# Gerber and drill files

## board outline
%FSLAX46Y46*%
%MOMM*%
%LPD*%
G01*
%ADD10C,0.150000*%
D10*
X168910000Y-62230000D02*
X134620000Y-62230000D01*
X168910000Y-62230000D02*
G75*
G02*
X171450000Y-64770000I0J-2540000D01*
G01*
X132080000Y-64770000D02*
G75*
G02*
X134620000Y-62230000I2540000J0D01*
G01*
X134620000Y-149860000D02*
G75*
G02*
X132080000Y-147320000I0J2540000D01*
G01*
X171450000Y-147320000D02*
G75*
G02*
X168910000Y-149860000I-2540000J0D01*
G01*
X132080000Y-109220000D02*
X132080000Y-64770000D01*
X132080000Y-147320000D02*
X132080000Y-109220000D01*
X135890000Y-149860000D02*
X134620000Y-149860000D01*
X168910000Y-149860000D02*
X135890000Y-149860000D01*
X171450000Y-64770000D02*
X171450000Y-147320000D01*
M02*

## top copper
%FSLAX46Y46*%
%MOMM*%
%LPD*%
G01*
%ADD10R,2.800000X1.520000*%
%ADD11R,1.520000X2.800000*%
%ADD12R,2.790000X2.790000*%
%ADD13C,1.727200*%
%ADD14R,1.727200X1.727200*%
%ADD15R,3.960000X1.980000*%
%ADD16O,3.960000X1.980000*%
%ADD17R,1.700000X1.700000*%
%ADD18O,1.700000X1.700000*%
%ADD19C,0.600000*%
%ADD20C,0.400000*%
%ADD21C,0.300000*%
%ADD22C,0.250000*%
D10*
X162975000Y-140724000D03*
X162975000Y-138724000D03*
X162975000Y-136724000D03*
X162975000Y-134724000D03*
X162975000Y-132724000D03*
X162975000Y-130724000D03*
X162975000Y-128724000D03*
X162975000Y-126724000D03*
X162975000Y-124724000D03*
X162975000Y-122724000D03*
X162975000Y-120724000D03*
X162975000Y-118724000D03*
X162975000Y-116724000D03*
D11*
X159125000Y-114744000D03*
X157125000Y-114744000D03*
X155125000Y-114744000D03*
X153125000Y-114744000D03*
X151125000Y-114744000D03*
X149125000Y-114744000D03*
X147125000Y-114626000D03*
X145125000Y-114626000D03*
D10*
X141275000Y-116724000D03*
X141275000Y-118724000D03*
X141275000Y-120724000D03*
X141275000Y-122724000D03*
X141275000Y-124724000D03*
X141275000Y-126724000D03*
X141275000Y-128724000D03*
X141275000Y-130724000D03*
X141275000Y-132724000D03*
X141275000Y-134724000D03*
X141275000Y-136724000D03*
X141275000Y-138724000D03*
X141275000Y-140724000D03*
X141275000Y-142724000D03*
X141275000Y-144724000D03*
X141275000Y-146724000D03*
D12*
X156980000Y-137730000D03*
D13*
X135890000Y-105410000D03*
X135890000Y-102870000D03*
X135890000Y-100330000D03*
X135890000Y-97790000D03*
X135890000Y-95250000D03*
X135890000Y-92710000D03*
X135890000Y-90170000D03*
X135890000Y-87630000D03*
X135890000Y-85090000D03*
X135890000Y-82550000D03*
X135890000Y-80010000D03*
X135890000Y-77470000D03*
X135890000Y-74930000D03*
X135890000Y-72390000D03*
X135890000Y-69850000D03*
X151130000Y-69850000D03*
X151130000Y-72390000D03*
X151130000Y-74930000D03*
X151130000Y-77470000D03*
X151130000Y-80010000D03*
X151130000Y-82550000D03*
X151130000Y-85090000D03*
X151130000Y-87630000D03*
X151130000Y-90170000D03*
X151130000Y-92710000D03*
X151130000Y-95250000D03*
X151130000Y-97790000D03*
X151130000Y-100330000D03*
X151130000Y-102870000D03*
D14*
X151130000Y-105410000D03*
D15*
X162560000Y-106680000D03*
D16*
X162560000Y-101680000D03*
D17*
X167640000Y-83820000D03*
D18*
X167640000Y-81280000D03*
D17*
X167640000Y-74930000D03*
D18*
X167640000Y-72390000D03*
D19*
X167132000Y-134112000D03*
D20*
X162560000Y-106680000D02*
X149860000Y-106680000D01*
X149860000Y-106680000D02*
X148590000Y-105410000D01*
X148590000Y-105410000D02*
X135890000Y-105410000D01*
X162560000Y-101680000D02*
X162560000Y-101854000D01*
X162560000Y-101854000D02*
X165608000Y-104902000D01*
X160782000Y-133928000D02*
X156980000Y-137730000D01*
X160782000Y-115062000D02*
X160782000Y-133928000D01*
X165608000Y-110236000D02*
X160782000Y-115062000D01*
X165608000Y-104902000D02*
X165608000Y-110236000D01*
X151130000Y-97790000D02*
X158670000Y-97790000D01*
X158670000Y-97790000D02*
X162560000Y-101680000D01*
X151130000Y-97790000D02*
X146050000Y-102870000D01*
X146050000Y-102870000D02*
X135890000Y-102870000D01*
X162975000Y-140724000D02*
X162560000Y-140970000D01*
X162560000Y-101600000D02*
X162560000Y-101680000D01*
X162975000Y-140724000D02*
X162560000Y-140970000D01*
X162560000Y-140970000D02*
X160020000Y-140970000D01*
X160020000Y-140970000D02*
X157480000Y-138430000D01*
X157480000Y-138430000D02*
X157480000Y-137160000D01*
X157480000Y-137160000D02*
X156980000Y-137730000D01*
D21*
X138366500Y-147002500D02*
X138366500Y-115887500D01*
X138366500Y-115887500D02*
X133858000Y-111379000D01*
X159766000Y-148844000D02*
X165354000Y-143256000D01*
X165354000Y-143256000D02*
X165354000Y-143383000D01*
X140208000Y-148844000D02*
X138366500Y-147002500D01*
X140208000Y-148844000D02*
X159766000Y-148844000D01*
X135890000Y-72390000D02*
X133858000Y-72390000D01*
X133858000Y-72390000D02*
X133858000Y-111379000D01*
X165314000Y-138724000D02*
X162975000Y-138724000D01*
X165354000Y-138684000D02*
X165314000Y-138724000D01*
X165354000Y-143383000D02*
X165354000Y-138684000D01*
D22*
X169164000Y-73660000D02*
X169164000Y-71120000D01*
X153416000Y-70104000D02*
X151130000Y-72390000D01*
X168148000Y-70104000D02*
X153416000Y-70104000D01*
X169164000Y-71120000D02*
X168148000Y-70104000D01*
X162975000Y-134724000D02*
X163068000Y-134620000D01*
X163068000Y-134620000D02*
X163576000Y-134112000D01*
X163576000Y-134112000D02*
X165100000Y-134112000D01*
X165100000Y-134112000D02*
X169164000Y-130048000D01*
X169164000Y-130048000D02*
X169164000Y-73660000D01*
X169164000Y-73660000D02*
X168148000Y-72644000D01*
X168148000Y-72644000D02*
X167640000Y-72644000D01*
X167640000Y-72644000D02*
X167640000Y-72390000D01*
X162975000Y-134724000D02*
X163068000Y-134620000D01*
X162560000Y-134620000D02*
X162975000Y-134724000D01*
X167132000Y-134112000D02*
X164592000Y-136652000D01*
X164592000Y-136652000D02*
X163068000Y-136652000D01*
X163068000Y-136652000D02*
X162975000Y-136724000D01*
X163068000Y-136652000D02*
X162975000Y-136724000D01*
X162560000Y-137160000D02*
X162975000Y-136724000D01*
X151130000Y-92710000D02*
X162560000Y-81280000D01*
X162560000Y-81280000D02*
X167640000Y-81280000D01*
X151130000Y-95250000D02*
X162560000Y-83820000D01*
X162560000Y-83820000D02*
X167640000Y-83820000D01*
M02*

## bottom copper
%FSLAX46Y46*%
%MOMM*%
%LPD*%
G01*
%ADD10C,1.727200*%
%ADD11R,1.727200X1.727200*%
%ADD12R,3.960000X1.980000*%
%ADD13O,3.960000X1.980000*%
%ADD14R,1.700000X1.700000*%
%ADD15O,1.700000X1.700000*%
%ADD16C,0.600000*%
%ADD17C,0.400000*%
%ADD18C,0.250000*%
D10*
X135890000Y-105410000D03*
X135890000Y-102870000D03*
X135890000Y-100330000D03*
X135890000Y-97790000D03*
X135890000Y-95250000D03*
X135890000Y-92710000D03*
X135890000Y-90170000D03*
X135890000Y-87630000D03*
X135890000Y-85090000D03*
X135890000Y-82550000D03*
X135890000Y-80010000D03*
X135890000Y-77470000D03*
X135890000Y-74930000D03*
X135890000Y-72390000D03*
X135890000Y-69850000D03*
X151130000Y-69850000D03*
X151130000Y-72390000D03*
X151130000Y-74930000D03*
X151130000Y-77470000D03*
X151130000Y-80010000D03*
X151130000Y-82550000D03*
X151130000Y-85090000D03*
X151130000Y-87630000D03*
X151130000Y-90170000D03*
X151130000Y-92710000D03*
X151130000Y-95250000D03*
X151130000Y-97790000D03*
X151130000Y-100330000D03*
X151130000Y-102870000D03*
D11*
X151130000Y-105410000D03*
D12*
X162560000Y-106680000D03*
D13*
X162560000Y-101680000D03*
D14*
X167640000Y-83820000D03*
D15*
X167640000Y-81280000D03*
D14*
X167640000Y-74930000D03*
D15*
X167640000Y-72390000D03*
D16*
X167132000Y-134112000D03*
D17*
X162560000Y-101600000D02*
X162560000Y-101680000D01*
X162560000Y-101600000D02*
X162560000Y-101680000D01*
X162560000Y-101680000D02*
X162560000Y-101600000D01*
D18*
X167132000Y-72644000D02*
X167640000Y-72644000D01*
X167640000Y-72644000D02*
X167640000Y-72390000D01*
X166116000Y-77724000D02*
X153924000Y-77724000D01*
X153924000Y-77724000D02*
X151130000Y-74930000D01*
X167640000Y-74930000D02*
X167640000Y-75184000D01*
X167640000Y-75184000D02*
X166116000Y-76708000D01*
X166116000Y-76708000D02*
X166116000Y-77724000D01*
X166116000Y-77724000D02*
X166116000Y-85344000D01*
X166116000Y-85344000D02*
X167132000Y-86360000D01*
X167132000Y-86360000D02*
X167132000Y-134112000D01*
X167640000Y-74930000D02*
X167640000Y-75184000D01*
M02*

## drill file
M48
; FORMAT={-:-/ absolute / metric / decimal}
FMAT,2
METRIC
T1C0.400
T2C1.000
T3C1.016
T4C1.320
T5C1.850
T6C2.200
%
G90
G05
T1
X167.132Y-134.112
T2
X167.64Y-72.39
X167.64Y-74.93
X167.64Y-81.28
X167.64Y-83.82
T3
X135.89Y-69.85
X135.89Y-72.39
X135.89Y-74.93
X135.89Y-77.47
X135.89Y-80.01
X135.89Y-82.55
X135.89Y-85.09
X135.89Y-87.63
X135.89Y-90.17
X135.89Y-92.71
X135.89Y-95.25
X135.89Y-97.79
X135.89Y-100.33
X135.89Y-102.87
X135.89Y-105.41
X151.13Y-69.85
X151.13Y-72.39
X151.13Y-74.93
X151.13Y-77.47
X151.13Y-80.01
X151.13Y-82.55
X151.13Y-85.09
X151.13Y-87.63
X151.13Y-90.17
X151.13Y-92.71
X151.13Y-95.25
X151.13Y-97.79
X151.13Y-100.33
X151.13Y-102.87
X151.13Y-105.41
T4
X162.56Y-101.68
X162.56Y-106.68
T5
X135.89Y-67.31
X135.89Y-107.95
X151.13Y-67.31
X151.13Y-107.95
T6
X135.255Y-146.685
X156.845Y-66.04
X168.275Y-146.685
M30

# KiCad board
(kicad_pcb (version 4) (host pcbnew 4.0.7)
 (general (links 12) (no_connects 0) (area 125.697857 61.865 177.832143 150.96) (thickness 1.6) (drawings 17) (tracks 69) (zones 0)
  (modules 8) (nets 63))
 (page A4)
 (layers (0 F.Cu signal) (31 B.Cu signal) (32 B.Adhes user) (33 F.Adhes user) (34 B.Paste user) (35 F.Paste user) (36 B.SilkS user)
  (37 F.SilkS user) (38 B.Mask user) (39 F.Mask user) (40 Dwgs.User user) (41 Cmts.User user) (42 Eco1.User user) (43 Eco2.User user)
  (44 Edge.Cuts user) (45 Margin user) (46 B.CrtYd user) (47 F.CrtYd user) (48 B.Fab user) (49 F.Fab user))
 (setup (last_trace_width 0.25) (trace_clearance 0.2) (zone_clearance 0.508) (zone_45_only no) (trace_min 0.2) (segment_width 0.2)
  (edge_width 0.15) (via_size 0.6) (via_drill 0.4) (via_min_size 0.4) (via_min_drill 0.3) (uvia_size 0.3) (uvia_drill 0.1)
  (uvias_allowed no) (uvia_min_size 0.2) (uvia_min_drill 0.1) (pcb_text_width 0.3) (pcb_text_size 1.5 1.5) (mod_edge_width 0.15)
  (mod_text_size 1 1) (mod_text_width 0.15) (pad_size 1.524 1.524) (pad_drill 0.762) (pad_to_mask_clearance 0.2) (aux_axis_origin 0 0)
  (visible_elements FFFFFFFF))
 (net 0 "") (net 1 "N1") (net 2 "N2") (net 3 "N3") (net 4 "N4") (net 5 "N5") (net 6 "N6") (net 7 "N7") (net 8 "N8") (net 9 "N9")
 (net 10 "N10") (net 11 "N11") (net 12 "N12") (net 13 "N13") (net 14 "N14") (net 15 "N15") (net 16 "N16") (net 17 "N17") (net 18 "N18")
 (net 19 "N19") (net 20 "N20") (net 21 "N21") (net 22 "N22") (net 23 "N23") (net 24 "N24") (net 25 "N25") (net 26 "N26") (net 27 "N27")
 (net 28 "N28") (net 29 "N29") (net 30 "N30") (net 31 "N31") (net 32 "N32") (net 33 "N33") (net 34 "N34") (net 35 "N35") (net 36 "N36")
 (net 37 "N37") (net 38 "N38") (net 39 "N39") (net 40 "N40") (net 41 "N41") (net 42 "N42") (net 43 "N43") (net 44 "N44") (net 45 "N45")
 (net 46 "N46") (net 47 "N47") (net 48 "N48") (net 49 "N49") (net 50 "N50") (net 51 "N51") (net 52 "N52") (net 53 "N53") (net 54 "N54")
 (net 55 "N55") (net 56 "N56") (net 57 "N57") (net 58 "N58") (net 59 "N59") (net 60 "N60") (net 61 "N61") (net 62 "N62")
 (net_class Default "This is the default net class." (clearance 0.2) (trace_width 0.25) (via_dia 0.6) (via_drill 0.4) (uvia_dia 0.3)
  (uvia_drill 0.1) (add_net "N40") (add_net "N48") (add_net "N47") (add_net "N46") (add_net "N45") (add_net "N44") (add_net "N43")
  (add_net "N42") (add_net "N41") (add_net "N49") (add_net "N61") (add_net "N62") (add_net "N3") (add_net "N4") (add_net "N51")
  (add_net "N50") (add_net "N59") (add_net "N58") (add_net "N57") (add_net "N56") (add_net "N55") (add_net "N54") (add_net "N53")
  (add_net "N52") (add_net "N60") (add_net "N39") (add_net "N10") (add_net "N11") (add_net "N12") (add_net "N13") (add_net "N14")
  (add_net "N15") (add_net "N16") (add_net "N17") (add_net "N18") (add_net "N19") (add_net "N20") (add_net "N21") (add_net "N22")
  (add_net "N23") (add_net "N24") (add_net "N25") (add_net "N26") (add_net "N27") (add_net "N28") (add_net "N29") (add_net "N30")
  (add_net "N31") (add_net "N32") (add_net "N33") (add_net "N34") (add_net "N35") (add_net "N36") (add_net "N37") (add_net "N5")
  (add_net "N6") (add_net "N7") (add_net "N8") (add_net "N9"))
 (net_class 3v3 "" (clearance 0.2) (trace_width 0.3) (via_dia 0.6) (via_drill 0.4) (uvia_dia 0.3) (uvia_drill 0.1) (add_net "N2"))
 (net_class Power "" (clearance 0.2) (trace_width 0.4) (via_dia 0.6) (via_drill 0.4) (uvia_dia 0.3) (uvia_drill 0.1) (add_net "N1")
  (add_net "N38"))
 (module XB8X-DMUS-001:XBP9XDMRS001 (layer F.Cu) (at 152.4 130.81 180)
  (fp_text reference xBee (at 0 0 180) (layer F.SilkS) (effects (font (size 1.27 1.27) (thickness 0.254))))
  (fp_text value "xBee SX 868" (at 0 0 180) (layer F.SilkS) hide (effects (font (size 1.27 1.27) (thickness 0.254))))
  (pad 1 smd rect (at -10.575 -9.914 270) (size 1.52 2.8) (layers F.Cu F.Paste F.Mask) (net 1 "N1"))
  (pad 2 smd rect (at -10.575 -7.914 270) (size 1.52 2.8) (layers F.Cu F.Paste F.Mask) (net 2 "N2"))
  (pad 3 smd rect (at -10.575 -5.914 270) (size 1.52 2.8) (layers F.Cu F.Paste F.Mask) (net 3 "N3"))
  (pad 4 smd rect (at -10.575 -3.914 270) (size 1.52 2.8) (layers F.Cu F.Paste F.Mask) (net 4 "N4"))
  (pad 5 smd rect (at -10.575 -1.914 270) (size 1.52 2.8) (layers F.Cu F.Paste F.Mask) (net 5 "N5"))
  (pad 6 smd rect (at -10.575 0.086 270) (size 1.52 2.8) (layers F.Cu F.Paste F.Mask) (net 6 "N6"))
  (pad 7 smd rect (at -10.575 2.086 270) (size 1.52 2.8) (layers F.Cu F.Paste F.Mask) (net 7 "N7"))
  (pad 8 smd rect (at -10.575 4.086 270) (size 1.52 2.8) (layers F.Cu F.Paste F.Mask) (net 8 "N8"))
  (pad 9 smd rect (at -10.575 6.086 270) (size 1.52 2.8) (layers F.Cu F.Paste F.Mask) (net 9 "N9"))
  (pad 10 smd rect (at -10.575 8.086 270) (size 1.52 2.8) (layers F.Cu F.Paste F.Mask) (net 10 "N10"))
  (pad 11 smd rect (at -10.575 10.086 270) (size 1.52 2.8) (layers F.Cu F.Paste F.Mask) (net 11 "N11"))
  (pad 12 smd rect (at -10.575 12.086 270) (size 1.52 2.8) (layers F.Cu F.Paste F.Mask) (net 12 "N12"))
  (pad 13 smd rect (at -10.575 14.086 270) (size 1.52 2.8) (layers F.Cu F.Paste F.Mask) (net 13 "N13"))
  (pad 14 smd rect (at -6.725 16.066 180) (size 1.52 2.8) (layers F.Cu F.Paste F.Mask) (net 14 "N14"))
  (pad 15 smd rect (at -4.725 16.066 180) (size 1.52 2.8) (layers F.Cu F.Paste F.Mask) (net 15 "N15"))
  (pad 16 smd rect (at -2.725 16.066 180) (size 1.52 2.8) (layers F.Cu F.Paste F.Mask) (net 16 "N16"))
  (pad 17 smd rect (at -0.725 16.066 180) (size 1.52 2.8) (layers F.Cu F.Paste F.Mask) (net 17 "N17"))
  (pad 18 smd rect (at 1.275 16.066 180) (size 1.52 2.8) (layers F.Cu F.Paste F.Mask) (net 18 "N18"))
  (pad 19 smd rect (at 3.275 16.066 180) (size 1.52 2.8) (layers F.Cu F.Paste F.Mask) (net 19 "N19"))
  (pad 20 smd rect (at 5.275 16.184 180) (size 1.52 2.8) (layers F.Cu F.Paste F.Mask) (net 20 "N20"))
  (pad 21 smd rect (at 7.275 16.184 180) (size 1.52 2.8) (layers F.Cu F.Paste F.Mask) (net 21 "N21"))
  (pad 22 smd rect (at 11.125 14.086 270) (size 1.52 2.8) (layers F.Cu F.Paste F.Mask) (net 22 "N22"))
  (pad 23 smd rect (at 11.125 12.086 270) (size 1.52 2.8) (layers F.Cu F.Paste F.Mask) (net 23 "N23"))
  (pad 24 smd rect (at 11.125 10.086 270) (size 1.52 2.8) (layers F.Cu F.Paste F.Mask) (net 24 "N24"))
  (pad 25 smd rect (at 11.125 8.086 270) (size 1.52 2.8) (layers F.Cu F.Paste F.Mask) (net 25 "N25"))
  (pad 26 smd rect (at 11.125 6.086 270) (size 1.52 2.8) (layers F.Cu F.Paste F.Mask) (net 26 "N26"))
  (pad 27 smd rect (at 11.125 4.086 270) (size 1.52 2.8) (layers F.Cu F.Paste F.Mask) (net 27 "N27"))
  (pad 28 smd rect (at 11.125 2.086 270) (size 1.52 2.8) (layers F.Cu F.Paste F.Mask) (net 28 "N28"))
  (pad 29 smd rect (at 11.125 0.086 270) (size 1.52 2.8) (layers F.Cu F.Paste F.Mask) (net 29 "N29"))
  (pad 30 smd rect (at 11.125 -1.914 270) (size 1.52 2.8) (layers F.Cu F.Paste F.Mask) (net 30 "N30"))
  (pad 31 smd rect (at 11.125 -3.914 270) (size 1.52 2.8) (layers F.Cu F.Paste F.Mask) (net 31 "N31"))
  (pad 32 smd rect (at 11.125 -5.914 270) (size 1.52 2.8) (layers F.Cu F.Paste F.Mask) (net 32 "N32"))
  (pad 33 smd rect (at 11.125 -7.914 270) (size 1.52 2.8) (layers F.Cu F.Paste F.Mask) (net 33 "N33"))
  (pad 34 smd rect (at 11.125 -9.914 270) (size 1.52 2.8) (layers F.Cu F.Paste F.Mask) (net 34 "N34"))
  (pad 35 smd rect (at 11.125 -11.914 270) (size 1.52 2.8) (layers F.Cu F.Paste F.Mask) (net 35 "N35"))
  (pad 36 smd rect (at 11.125 -13.914 270) (size 1.52 2.8) (layers F.Cu F.Paste F.Mask) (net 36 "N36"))
  (pad 37 smd rect (at 11.125 -15.914 270) (size 1.52 2.8) (layers F.Cu F.Paste F.Mask) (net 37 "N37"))
  (pad 38 smd rect (at -4.58 -6.92 180) (size 2.79 2.79) (layers F.Cu F.Paste F.Mask) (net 1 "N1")))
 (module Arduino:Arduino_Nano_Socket (layer F.Cu) (at 143.51 66.04 180)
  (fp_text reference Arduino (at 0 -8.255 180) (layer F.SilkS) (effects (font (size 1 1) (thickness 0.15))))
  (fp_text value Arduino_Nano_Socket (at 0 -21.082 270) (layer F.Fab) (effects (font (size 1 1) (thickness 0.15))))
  (pad VIN thru_hole circle (at 7.62 -39.37 180) (size 1.7272 1.7272) (drill 1.016) (layers *.Cu *.Mask) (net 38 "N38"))
  (pad GND2 thru_hole circle (at 7.62 -36.83 180) (size 1.7272 1.7272) (drill 1.016) (layers *.Cu *.Mask) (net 1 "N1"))
  (pad RST2 thru_hole circle (at 7.62 -34.29 180) (size 1.7272 1.7272) (drill 1.016) (layers *.Cu *.Mask) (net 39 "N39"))
  (pad 5V thru_hole circle (at 7.62 -31.75 180) (size 1.7272 1.7272) (drill 1.016) (layers *.Cu *.Mask) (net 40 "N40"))
  (pad A7 thru_hole circle (at 7.62 -29.21 180) (size 1.7272 1.7272) (drill 1.016) (layers *.Cu *.Mask) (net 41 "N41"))
  (pad A6 thru_hole circle (at 7.62 -26.67 180) (size 1.7272 1.7272) (drill 1.016) (layers *.Cu *.Mask) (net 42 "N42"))
  (pad A5 thru_hole circle (at 7.62 -24.13 180) (size 1.7272 1.7272) (drill 1.016) (layers *.Cu *.Mask) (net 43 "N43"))
  (pad A4 thru_hole circle (at 7.62 -21.59 180) (size 1.7272 1.7272) (drill 1.016) (layers *.Cu *.Mask) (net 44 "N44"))
  (pad A3 thru_hole circle (at 7.62 -19.05 180) (size 1.7272 1.7272) (drill 1.016) (layers *.Cu *.Mask) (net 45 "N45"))
  (pad A2 thru_hole circle (at 7.62 -16.51 180) (size 1.7272 1.7272) (drill 1.016) (layers *.Cu *.Mask) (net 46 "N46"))
  (pad A1 thru_hole circle (at 7.62 -13.97 180) (size 1.7272 1.7272) (drill 1.016) (layers *.Cu *.Mask) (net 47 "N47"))
  (pad A0 thru_hole circle (at 7.62 -11.43 180) (size 1.7272 1.7272) (drill 1.016) (layers *.Cu *.Mask) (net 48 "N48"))
  (pad AREF thru_hole circle (at 7.62 -8.89 180) (size 1.7272 1.7272) (drill 1.016) (layers *.Cu *.Mask) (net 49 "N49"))
  (pad 3V3 thru_hole circle (at 7.62 -6.35 180) (size 1.7272 1.7272) (drill 1.016) (layers *.Cu *.Mask) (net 2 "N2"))
  (pad D13 thru_hole circle (at 7.62 -3.81 180) (size 1.7272 1.7272) (drill 1.016) (layers *.Cu *.Mask) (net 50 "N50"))
  (pad D12 thru_hole circle (at -7.62 -3.81 180) (size 1.7272 1.7272) (drill 1.016) (layers *.Cu *.Mask) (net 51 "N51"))
  (pad D11 thru_hole circle (at -7.62 -6.35 180) (size 1.7272 1.7272) (drill 1.016) (layers *.Cu *.Mask) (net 4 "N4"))
  (pad D10 thru_hole circle (at -7.62 -8.89 180) (size 1.7272 1.7272) (drill 1.016) (layers *.Cu *.Mask) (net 3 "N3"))
  (pad D9 thru_hole circle (at -7.62 -11.43 180) (size 1.7272 1.7272) (drill 1.016) (layers *.Cu *.Mask) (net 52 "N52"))
  (pad D8 thru_hole circle (at -7.62 -13.97 180) (size 1.7272 1.7272) (drill 1.016) (layers *.Cu *.Mask) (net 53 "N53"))
  (pad D7 thru_hole circle (at -7.62 -16.51 180) (size 1.7272 1.7272) (drill 1.016) (layers *.Cu *.Mask) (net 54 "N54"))
  (pad D6 thru_hole circle (at -7.62 -19.05 180) (size 1.7272 1.7272) (drill 1.016) (layers *.Cu *.Mask) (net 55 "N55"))
  (pad D5 thru_hole circle (at -7.62 -21.59 180) (size 1.7272 1.7272) (drill 1.016) (layers *.Cu *.Mask) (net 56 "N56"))
  (pad D4 thru_hole circle (at -7.62 -24.13 180) (size 1.7272 1.7272) (drill 1.016) (layers *.Cu *.Mask) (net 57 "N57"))
  (pad D3 thru_hole circle (at -7.62 -26.67 180) (size 1.7272 1.7272) (drill 1.016) (layers *.Cu *.Mask) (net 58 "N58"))
  (pad D2 thru_hole circle (at -7.62 -29.21 180) (size 1.7272 1.7272) (drill 1.016) (layers *.Cu *.Mask) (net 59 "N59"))
  (pad GND1 thru_hole circle (at -7.62 -31.75 180) (size 1.7272 1.7272) (drill 1.016) (layers *.Cu *.Mask) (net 1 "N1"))
  (pad RST1 thru_hole circle (at -7.62 -34.29 180) (size 1.7272 1.7272) (drill 1.016) (layers *.Cu *.Mask) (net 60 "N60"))
  (pad D0 thru_hole circle (at -7.62 -36.83 180) (size 1.7272 1.7272) (drill 1.016) (layers *.Cu *.Mask) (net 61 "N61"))
  (pad D1 thru_hole rect (at -7.62 -39.37 180) (size 1.7272 1.7272) (drill 1.016) (layers *.Cu *.Mask) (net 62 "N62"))
  (pad "" np_thru_hole circle (at -7.62 -41.91 180) (size 1.85 1.85) (drill 1.85) (layers *.Cu *.Mask))
  (pad "" np_thru_hole circle (at 7.62 -41.91 180) (size 1.85 1.85) (drill 1.85) (layers *.Cu *.Mask))
  (pad "" np_thru_hole circle (at -7.62 -1.27 180) (size 1.85 1.85) (drill 1.85) (layers *.Cu *.Mask))
  (pad "" np_thru_hole circle (at 7.62 -1.27 180) (size 1.85 1.85) (drill 1.85) (layers *.Cu *.Mask)))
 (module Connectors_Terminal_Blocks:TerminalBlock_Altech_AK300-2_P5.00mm (layer F.Cu) (at 162.56 106.68 90)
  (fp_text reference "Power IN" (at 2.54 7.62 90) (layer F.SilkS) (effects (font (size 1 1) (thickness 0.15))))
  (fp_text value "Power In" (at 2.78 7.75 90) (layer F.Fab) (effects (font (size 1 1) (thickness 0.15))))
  (pad 1 thru_hole rect (at 0 0 90) (size 1.98 3.96) (drill 1.32) (layers *.Cu *.Mask) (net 38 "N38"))
  (pad 2 thru_hole oval (at 5 0 90) (size 1.98 3.96) (drill 1.32) (layers *.Cu *.Mask) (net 1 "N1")))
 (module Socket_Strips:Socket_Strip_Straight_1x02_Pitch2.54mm (layer F.Cu) (at 167.64 83.82 180)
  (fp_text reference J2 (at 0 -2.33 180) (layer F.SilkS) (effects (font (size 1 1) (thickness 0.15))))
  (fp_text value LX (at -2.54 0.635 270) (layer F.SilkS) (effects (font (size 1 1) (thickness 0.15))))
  (pad 1 thru_hole rect (at 0 0 180) (size 1.7 1.7) (drill 1) (layers *.Cu *.Mask) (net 59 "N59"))
  (pad 2 thru_hole oval (at 0 2.54 180) (size 1.7 1.7) (drill 1) (layers *.Cu *.Mask) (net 58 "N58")))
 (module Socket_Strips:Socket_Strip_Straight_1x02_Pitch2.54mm (layer F.Cu) (at 167.64 74.93 180)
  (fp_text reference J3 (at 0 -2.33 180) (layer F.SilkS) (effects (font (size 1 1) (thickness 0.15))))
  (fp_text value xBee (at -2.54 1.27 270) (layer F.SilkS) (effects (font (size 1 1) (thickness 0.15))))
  (pad 1 thru_hole rect (at 0 0 180) (size 1.7 1.7) (drill 1) (layers *.Cu *.Mask) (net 3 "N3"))
  (pad 2 thru_hole oval (at 0 2.54 180) (size 1.7 1.7) (drill 1) (layers *.Cu *.Mask) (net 4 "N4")))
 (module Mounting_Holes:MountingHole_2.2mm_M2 (layer F.Cu) (at 168.275 146.685)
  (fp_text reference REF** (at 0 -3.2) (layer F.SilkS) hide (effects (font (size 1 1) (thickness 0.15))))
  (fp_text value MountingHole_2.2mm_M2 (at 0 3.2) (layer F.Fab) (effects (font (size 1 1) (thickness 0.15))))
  (pad 1 np_thru_hole circle (at 0 0) (size 2.2 2.2) (drill 2.2) (layers *.Cu *.Mask)))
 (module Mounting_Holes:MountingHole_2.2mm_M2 (layer F.Cu) (at 135.255 146.685)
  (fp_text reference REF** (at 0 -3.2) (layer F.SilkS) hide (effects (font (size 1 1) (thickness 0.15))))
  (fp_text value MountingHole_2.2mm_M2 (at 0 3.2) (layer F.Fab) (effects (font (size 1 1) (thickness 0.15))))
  (pad 1 np_thru_hole circle (at 0 0) (size 2.2 2.2) (drill 2.2) (layers *.Cu *.Mask)))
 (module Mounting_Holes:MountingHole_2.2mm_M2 (layer F.Cu) (at 156.845 66.04)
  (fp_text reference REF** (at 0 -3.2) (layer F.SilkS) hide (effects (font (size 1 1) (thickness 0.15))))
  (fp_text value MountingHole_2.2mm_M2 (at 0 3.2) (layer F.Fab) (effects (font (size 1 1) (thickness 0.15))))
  (pad 1 np_thru_hole circle (at 0 0) (size 2.2 2.2) (drill 2.2) (layers *.Cu *.Mask)))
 (gr_line (start 168.91 62.23) (end 134.62 62.23) (angle 90) (layer Edge.Cuts) (width 0.15))
 (gr_arc (start 168.91 64.77) (end 168.91 62.23) (angle 90) (layer Edge.Cuts) (width 0.15))
 (gr_arc (start 134.62 64.77) (end 132.08 64.77) (angle 90) (layer Edge.Cuts) (width 0.15))
 (gr_arc (start 134.62 147.32) (end 134.62 149.86) (angle 90) (layer Edge.Cuts) (width 0.15))
 (gr_arc (start 168.91 147.32) (end 171.45 147.32) (angle 90) (layer Edge.Cuts) (width 0.15))
 (gr_line (start 132.08 109.22) (end 132.08 64.77) (angle 90) (layer Edge.Cuts) (width 0.15))
 (gr_line (start 132.08 147.32) (end 132.08 109.22) (angle 90) (layer Edge.Cuts) (width 0.15))
 (gr_line (start 135.89 149.86) (end 134.62 149.86) (angle 90) (layer Edge.Cuts) (width 0.15))
 (gr_line (start 168.91 149.86) (end 135.89 149.86) (angle 90) (layer Edge.Cuts) (width 0.15))
 (gr_line (start 171.45 64.77) (end 171.45 147.32) (angle 90) (layer Edge.Cuts) (width 0.15))
 (segment (start 162.56 106.68) (end 149.86 106.68) (width 0.4) (layer F.Cu) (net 38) (status 80000))
 (segment (start 149.86 106.68) (end 148.59 105.41) (width 0.4) (layer F.Cu) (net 38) (status 80000))
 (segment (start 148.59 105.41) (end 135.89 105.41) (width 0.4) (layer F.Cu) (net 38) (status 80000))
 (segment (start 162.56 101.68) (end 162.56 101.854) (width 0.4) (layer F.Cu) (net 1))
 (segment (start 162.56 101.854) (end 165.608 104.902) (width 0.4) (layer F.Cu) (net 1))
 (segment (start 160.782 133.928) (end 156.98 137.73) (width 0.4) (layer F.Cu) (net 1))
 (segment (start 160.782 115.062) (end 160.782 133.928) (width 0.4) (layer F.Cu) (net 1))
 (segment (start 165.608 110.236) (end 160.782 115.062) (width 0.4) (layer F.Cu) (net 1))
 (segment (start 165.608 104.902) (end 165.608 110.236) (width 0.4) (layer F.Cu) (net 1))
 (segment (start 151.13 97.79) (end 158.67 97.79) (width 0.4) (layer F.Cu) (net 1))
 (segment (start 158.67 97.79) (end 162.56 101.68) (width 0.4) (layer F.Cu) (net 1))
 (segment (start 162.56 101.6) (end 162.56 101.68) (width 0.4) (layer B.Cu) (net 1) (status 80000))
 (segment (start 151.13 97.79) (end 146.05 102.87) (width 0.4) (layer F.Cu) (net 1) (status 80000))
 (segment (start 146.05 102.87) (end 135.89 102.87) (width 0.4) (layer F.Cu) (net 1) (status 80000))
 (segment (start 162.56 101.6) (end 162.56 101.68) (width 0.4) (layer B.Cu) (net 1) (status 80000))
 (segment (start 162.975 140.724) (end 162.56 140.97) (width 0.4) (layer F.Cu) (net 1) (status 80000))
 (segment (start 162.56 101.6) (end 162.56 101.68) (width 0.4) (layer F.Cu) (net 1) (status 80000))
 (segment (start 162.56 101.68) (end 162.56 101.6) (width 0.4) (layer B.Cu) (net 1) (status 80000))
 (segment (start 162.975 140.724) (end 162.56 140.97) (width 0.4) (layer F.Cu) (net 1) (status 80000))
 (segment (start 162.56 140.97) (end 160.02 140.97) (width 0.4) (layer F.Cu) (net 1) (status 80000))
 (segment (start 160.02 140.97) (end 157.48 138.43) (width 0.4) (layer F.Cu) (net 1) (status 80000))
 (segment (start 157.48 138.43) (end 157.48 137.16) (width 0.4) (layer F.Cu) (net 1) (status 80000))
 (segment (start 157.48 137.16) (end 156.98 137.73) (width 0.4) (layer F.Cu) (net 1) (status 80000))
 (segment (start 138.3665 147.0025) (end 138.3665 115.8875) (width 0.3) (layer F.Cu) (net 2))
 (segment (start 138.3665 115.8875) (end 133.858 111.379) (width 0.3) (layer F.Cu) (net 2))
 (segment (start 159.766 148.844) (end 165.354 143.256) (width 0.3) (layer F.Cu) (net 2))
 (segment (start 165.354 143.256) (end 165.354 143.383) (width 0.3) (layer F.Cu) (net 2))
 (segment (start 140.208 148.844) (end 138.3665 147.0025) (width 0.3) (layer F.Cu) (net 2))
 (segment (start 140.208 148.844) (end 159.766 148.844) (width 0.3) (layer F.Cu) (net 2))
 (segment (start 135.89 72.39) (end 133.858 72.39) (width 0.3) (layer F.Cu) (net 2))
 (segment (start 133.858 72.39) (end 133.858 111.379) (width 0.3) (layer F.Cu) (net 2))
 (segment (start 165.314 138.724) (end 162.975 138.724) (width 0.3) (layer F.Cu) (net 2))
 (segment (start 165.354 138.684) (end 165.314 138.724) (width 0.3) (layer F.Cu) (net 2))
 (segment (start 165.354 143.383) (end 165.354 138.684) (width 0.3) (layer F.Cu) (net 2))
 (segment (start 169.164 73.66) (end 169.164 71.12) (width 0.25) (layer F.Cu) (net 4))
 (segment (start 153.416 70.104) (end 151.13 72.39) (width 0.25) (layer F.Cu) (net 4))
 (segment (start 168.148 70.104) (end 153.416 70.104) (width 0.25) (layer F.Cu) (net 4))
 (segment (start 169.164 71.12) (end 168.148 70.104) (width 0.25) (layer F.Cu) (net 4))
 (segment (start 162.975 134.724) (end 163.068 134.62) (width 0.25) (layer F.Cu) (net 4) (status 80000))
 (segment (start 163.068 134.62) (end 163.576 134.112) (width 0.25) (layer F.Cu) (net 4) (status 80000))
 (segment (start 163.576 134.112) (end 165.1 134.112) (width 0.25) (layer F.Cu) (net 4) (status 80000))
 (segment (start 165.1 134.112) (end 169.164 130.048) (width 0.25) (layer F.Cu) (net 4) (status 80000))
 (segment (start 169.164 130.048) (end 169.164 73.66) (width 0.25) (layer F.Cu) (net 4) (status 80000))
 (segment (start 169.164 73.66) (end 168.148 72.644) (width 0.25) (layer F.Cu) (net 4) (status 80000))
 (segment (start 168.148 72.644) (end 167.64 72.644) (width 0.25) (layer F.Cu) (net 4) (status 80000))
 (segment (start 167.64 72.644) (end 167.64 72.39) (width 0.25) (layer F.Cu) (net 4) (status 80000))
 (segment (start 162.975 134.724) (end 163.068 134.62) (width 0.25) (layer F.Cu) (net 4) (status 80000))
 (segment (start 167.132 72.644) (end 167.64 72.644) (width 0.25) (layer B.Cu) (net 4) (status 80000))
 (segment (start 167.64 72.644) (end 167.64 72.39) (width 0.25) (layer B.Cu) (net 4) (status 80000))
 (segment (start 162.56 134.62) (end 162.975 134.724) (width 0.25) (layer F.Cu) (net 4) (status 80000))
 (segment (start 166.116 77.724) (end 153.924 77.724) (width 0.25) (layer B.Cu) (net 3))
 (segment (start 153.924 77.724) (end 151.13 74.93) (width 0.25) (layer B.Cu) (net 3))
 (segment (start 167.64 74.93) (end 167.64 75.184) (width 0.25) (layer B.Cu) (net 3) (status 80000))
 (segment (start 167.64 75.184) (end 166.116 76.708) (width 0.25) (layer B.Cu) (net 3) (status 80000))
 (segment (start 166.116 76.708) (end 166.116 77.724) (width 0.25) (layer B.Cu) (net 3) (status 80000))
 (segment (start 166.116 77.724) (end 166.116 85.344) (width 0.25) (layer B.Cu) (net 3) (status 80000))
 (segment (start 166.116 85.344) (end 167.132 86.36) (width 0.25) (layer B.Cu) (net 3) (status 80000))
 (segment (start 167.132 86.36) (end 167.132 134.112) (width 0.25) (layer B.Cu) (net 3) (status 80000))
 (via (at 167.132 134.112) (size 0.6) (layers F.Cu B.Cu) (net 3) (status 80000))
 (segment (start 167.132 134.112) (end 164.592 136.652) (width 0.25) (layer F.Cu) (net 3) (status 80000))
 (segment (start 164.592 136.652) (end 163.068 136.652) (width 0.25) (layer F.Cu) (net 3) (status 80000))
 (segment (start 163.068 136.652) (end 162.975 136.724) (width 0.25) (layer F.Cu) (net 3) (status 80000))
 (segment (start 167.64 74.93) (end 167.64 75.184) (width 0.25) (layer B.Cu) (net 3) (status 80000))
 (segment (start 163.068 136.652) (end 162.975 136.724) (width 0.25) (layer F.Cu) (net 3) (status 80000))
 (segment (start 162.56 137.16) (end 162.975 136.724) (width 0.25) (layer F.Cu) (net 3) (status 80000))
 (segment (start 151.13 92.71) (end 162.56 81.28) (width 0.25) (layer F.Cu) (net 58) (status 80000))
 (segment (start 162.56 81.28) (end 167.64 81.28) (width 0.25) (layer F.Cu) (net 58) (status 80000))
 (segment (start 151.13 95.25) (end 162.56 83.82) (width 0.25) (layer F.Cu) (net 59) (status 80000))
 (segment (start 162.56 83.82) (end 167.64 83.82) (width 0.25) (layer F.Cu) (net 59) (status 80000)))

